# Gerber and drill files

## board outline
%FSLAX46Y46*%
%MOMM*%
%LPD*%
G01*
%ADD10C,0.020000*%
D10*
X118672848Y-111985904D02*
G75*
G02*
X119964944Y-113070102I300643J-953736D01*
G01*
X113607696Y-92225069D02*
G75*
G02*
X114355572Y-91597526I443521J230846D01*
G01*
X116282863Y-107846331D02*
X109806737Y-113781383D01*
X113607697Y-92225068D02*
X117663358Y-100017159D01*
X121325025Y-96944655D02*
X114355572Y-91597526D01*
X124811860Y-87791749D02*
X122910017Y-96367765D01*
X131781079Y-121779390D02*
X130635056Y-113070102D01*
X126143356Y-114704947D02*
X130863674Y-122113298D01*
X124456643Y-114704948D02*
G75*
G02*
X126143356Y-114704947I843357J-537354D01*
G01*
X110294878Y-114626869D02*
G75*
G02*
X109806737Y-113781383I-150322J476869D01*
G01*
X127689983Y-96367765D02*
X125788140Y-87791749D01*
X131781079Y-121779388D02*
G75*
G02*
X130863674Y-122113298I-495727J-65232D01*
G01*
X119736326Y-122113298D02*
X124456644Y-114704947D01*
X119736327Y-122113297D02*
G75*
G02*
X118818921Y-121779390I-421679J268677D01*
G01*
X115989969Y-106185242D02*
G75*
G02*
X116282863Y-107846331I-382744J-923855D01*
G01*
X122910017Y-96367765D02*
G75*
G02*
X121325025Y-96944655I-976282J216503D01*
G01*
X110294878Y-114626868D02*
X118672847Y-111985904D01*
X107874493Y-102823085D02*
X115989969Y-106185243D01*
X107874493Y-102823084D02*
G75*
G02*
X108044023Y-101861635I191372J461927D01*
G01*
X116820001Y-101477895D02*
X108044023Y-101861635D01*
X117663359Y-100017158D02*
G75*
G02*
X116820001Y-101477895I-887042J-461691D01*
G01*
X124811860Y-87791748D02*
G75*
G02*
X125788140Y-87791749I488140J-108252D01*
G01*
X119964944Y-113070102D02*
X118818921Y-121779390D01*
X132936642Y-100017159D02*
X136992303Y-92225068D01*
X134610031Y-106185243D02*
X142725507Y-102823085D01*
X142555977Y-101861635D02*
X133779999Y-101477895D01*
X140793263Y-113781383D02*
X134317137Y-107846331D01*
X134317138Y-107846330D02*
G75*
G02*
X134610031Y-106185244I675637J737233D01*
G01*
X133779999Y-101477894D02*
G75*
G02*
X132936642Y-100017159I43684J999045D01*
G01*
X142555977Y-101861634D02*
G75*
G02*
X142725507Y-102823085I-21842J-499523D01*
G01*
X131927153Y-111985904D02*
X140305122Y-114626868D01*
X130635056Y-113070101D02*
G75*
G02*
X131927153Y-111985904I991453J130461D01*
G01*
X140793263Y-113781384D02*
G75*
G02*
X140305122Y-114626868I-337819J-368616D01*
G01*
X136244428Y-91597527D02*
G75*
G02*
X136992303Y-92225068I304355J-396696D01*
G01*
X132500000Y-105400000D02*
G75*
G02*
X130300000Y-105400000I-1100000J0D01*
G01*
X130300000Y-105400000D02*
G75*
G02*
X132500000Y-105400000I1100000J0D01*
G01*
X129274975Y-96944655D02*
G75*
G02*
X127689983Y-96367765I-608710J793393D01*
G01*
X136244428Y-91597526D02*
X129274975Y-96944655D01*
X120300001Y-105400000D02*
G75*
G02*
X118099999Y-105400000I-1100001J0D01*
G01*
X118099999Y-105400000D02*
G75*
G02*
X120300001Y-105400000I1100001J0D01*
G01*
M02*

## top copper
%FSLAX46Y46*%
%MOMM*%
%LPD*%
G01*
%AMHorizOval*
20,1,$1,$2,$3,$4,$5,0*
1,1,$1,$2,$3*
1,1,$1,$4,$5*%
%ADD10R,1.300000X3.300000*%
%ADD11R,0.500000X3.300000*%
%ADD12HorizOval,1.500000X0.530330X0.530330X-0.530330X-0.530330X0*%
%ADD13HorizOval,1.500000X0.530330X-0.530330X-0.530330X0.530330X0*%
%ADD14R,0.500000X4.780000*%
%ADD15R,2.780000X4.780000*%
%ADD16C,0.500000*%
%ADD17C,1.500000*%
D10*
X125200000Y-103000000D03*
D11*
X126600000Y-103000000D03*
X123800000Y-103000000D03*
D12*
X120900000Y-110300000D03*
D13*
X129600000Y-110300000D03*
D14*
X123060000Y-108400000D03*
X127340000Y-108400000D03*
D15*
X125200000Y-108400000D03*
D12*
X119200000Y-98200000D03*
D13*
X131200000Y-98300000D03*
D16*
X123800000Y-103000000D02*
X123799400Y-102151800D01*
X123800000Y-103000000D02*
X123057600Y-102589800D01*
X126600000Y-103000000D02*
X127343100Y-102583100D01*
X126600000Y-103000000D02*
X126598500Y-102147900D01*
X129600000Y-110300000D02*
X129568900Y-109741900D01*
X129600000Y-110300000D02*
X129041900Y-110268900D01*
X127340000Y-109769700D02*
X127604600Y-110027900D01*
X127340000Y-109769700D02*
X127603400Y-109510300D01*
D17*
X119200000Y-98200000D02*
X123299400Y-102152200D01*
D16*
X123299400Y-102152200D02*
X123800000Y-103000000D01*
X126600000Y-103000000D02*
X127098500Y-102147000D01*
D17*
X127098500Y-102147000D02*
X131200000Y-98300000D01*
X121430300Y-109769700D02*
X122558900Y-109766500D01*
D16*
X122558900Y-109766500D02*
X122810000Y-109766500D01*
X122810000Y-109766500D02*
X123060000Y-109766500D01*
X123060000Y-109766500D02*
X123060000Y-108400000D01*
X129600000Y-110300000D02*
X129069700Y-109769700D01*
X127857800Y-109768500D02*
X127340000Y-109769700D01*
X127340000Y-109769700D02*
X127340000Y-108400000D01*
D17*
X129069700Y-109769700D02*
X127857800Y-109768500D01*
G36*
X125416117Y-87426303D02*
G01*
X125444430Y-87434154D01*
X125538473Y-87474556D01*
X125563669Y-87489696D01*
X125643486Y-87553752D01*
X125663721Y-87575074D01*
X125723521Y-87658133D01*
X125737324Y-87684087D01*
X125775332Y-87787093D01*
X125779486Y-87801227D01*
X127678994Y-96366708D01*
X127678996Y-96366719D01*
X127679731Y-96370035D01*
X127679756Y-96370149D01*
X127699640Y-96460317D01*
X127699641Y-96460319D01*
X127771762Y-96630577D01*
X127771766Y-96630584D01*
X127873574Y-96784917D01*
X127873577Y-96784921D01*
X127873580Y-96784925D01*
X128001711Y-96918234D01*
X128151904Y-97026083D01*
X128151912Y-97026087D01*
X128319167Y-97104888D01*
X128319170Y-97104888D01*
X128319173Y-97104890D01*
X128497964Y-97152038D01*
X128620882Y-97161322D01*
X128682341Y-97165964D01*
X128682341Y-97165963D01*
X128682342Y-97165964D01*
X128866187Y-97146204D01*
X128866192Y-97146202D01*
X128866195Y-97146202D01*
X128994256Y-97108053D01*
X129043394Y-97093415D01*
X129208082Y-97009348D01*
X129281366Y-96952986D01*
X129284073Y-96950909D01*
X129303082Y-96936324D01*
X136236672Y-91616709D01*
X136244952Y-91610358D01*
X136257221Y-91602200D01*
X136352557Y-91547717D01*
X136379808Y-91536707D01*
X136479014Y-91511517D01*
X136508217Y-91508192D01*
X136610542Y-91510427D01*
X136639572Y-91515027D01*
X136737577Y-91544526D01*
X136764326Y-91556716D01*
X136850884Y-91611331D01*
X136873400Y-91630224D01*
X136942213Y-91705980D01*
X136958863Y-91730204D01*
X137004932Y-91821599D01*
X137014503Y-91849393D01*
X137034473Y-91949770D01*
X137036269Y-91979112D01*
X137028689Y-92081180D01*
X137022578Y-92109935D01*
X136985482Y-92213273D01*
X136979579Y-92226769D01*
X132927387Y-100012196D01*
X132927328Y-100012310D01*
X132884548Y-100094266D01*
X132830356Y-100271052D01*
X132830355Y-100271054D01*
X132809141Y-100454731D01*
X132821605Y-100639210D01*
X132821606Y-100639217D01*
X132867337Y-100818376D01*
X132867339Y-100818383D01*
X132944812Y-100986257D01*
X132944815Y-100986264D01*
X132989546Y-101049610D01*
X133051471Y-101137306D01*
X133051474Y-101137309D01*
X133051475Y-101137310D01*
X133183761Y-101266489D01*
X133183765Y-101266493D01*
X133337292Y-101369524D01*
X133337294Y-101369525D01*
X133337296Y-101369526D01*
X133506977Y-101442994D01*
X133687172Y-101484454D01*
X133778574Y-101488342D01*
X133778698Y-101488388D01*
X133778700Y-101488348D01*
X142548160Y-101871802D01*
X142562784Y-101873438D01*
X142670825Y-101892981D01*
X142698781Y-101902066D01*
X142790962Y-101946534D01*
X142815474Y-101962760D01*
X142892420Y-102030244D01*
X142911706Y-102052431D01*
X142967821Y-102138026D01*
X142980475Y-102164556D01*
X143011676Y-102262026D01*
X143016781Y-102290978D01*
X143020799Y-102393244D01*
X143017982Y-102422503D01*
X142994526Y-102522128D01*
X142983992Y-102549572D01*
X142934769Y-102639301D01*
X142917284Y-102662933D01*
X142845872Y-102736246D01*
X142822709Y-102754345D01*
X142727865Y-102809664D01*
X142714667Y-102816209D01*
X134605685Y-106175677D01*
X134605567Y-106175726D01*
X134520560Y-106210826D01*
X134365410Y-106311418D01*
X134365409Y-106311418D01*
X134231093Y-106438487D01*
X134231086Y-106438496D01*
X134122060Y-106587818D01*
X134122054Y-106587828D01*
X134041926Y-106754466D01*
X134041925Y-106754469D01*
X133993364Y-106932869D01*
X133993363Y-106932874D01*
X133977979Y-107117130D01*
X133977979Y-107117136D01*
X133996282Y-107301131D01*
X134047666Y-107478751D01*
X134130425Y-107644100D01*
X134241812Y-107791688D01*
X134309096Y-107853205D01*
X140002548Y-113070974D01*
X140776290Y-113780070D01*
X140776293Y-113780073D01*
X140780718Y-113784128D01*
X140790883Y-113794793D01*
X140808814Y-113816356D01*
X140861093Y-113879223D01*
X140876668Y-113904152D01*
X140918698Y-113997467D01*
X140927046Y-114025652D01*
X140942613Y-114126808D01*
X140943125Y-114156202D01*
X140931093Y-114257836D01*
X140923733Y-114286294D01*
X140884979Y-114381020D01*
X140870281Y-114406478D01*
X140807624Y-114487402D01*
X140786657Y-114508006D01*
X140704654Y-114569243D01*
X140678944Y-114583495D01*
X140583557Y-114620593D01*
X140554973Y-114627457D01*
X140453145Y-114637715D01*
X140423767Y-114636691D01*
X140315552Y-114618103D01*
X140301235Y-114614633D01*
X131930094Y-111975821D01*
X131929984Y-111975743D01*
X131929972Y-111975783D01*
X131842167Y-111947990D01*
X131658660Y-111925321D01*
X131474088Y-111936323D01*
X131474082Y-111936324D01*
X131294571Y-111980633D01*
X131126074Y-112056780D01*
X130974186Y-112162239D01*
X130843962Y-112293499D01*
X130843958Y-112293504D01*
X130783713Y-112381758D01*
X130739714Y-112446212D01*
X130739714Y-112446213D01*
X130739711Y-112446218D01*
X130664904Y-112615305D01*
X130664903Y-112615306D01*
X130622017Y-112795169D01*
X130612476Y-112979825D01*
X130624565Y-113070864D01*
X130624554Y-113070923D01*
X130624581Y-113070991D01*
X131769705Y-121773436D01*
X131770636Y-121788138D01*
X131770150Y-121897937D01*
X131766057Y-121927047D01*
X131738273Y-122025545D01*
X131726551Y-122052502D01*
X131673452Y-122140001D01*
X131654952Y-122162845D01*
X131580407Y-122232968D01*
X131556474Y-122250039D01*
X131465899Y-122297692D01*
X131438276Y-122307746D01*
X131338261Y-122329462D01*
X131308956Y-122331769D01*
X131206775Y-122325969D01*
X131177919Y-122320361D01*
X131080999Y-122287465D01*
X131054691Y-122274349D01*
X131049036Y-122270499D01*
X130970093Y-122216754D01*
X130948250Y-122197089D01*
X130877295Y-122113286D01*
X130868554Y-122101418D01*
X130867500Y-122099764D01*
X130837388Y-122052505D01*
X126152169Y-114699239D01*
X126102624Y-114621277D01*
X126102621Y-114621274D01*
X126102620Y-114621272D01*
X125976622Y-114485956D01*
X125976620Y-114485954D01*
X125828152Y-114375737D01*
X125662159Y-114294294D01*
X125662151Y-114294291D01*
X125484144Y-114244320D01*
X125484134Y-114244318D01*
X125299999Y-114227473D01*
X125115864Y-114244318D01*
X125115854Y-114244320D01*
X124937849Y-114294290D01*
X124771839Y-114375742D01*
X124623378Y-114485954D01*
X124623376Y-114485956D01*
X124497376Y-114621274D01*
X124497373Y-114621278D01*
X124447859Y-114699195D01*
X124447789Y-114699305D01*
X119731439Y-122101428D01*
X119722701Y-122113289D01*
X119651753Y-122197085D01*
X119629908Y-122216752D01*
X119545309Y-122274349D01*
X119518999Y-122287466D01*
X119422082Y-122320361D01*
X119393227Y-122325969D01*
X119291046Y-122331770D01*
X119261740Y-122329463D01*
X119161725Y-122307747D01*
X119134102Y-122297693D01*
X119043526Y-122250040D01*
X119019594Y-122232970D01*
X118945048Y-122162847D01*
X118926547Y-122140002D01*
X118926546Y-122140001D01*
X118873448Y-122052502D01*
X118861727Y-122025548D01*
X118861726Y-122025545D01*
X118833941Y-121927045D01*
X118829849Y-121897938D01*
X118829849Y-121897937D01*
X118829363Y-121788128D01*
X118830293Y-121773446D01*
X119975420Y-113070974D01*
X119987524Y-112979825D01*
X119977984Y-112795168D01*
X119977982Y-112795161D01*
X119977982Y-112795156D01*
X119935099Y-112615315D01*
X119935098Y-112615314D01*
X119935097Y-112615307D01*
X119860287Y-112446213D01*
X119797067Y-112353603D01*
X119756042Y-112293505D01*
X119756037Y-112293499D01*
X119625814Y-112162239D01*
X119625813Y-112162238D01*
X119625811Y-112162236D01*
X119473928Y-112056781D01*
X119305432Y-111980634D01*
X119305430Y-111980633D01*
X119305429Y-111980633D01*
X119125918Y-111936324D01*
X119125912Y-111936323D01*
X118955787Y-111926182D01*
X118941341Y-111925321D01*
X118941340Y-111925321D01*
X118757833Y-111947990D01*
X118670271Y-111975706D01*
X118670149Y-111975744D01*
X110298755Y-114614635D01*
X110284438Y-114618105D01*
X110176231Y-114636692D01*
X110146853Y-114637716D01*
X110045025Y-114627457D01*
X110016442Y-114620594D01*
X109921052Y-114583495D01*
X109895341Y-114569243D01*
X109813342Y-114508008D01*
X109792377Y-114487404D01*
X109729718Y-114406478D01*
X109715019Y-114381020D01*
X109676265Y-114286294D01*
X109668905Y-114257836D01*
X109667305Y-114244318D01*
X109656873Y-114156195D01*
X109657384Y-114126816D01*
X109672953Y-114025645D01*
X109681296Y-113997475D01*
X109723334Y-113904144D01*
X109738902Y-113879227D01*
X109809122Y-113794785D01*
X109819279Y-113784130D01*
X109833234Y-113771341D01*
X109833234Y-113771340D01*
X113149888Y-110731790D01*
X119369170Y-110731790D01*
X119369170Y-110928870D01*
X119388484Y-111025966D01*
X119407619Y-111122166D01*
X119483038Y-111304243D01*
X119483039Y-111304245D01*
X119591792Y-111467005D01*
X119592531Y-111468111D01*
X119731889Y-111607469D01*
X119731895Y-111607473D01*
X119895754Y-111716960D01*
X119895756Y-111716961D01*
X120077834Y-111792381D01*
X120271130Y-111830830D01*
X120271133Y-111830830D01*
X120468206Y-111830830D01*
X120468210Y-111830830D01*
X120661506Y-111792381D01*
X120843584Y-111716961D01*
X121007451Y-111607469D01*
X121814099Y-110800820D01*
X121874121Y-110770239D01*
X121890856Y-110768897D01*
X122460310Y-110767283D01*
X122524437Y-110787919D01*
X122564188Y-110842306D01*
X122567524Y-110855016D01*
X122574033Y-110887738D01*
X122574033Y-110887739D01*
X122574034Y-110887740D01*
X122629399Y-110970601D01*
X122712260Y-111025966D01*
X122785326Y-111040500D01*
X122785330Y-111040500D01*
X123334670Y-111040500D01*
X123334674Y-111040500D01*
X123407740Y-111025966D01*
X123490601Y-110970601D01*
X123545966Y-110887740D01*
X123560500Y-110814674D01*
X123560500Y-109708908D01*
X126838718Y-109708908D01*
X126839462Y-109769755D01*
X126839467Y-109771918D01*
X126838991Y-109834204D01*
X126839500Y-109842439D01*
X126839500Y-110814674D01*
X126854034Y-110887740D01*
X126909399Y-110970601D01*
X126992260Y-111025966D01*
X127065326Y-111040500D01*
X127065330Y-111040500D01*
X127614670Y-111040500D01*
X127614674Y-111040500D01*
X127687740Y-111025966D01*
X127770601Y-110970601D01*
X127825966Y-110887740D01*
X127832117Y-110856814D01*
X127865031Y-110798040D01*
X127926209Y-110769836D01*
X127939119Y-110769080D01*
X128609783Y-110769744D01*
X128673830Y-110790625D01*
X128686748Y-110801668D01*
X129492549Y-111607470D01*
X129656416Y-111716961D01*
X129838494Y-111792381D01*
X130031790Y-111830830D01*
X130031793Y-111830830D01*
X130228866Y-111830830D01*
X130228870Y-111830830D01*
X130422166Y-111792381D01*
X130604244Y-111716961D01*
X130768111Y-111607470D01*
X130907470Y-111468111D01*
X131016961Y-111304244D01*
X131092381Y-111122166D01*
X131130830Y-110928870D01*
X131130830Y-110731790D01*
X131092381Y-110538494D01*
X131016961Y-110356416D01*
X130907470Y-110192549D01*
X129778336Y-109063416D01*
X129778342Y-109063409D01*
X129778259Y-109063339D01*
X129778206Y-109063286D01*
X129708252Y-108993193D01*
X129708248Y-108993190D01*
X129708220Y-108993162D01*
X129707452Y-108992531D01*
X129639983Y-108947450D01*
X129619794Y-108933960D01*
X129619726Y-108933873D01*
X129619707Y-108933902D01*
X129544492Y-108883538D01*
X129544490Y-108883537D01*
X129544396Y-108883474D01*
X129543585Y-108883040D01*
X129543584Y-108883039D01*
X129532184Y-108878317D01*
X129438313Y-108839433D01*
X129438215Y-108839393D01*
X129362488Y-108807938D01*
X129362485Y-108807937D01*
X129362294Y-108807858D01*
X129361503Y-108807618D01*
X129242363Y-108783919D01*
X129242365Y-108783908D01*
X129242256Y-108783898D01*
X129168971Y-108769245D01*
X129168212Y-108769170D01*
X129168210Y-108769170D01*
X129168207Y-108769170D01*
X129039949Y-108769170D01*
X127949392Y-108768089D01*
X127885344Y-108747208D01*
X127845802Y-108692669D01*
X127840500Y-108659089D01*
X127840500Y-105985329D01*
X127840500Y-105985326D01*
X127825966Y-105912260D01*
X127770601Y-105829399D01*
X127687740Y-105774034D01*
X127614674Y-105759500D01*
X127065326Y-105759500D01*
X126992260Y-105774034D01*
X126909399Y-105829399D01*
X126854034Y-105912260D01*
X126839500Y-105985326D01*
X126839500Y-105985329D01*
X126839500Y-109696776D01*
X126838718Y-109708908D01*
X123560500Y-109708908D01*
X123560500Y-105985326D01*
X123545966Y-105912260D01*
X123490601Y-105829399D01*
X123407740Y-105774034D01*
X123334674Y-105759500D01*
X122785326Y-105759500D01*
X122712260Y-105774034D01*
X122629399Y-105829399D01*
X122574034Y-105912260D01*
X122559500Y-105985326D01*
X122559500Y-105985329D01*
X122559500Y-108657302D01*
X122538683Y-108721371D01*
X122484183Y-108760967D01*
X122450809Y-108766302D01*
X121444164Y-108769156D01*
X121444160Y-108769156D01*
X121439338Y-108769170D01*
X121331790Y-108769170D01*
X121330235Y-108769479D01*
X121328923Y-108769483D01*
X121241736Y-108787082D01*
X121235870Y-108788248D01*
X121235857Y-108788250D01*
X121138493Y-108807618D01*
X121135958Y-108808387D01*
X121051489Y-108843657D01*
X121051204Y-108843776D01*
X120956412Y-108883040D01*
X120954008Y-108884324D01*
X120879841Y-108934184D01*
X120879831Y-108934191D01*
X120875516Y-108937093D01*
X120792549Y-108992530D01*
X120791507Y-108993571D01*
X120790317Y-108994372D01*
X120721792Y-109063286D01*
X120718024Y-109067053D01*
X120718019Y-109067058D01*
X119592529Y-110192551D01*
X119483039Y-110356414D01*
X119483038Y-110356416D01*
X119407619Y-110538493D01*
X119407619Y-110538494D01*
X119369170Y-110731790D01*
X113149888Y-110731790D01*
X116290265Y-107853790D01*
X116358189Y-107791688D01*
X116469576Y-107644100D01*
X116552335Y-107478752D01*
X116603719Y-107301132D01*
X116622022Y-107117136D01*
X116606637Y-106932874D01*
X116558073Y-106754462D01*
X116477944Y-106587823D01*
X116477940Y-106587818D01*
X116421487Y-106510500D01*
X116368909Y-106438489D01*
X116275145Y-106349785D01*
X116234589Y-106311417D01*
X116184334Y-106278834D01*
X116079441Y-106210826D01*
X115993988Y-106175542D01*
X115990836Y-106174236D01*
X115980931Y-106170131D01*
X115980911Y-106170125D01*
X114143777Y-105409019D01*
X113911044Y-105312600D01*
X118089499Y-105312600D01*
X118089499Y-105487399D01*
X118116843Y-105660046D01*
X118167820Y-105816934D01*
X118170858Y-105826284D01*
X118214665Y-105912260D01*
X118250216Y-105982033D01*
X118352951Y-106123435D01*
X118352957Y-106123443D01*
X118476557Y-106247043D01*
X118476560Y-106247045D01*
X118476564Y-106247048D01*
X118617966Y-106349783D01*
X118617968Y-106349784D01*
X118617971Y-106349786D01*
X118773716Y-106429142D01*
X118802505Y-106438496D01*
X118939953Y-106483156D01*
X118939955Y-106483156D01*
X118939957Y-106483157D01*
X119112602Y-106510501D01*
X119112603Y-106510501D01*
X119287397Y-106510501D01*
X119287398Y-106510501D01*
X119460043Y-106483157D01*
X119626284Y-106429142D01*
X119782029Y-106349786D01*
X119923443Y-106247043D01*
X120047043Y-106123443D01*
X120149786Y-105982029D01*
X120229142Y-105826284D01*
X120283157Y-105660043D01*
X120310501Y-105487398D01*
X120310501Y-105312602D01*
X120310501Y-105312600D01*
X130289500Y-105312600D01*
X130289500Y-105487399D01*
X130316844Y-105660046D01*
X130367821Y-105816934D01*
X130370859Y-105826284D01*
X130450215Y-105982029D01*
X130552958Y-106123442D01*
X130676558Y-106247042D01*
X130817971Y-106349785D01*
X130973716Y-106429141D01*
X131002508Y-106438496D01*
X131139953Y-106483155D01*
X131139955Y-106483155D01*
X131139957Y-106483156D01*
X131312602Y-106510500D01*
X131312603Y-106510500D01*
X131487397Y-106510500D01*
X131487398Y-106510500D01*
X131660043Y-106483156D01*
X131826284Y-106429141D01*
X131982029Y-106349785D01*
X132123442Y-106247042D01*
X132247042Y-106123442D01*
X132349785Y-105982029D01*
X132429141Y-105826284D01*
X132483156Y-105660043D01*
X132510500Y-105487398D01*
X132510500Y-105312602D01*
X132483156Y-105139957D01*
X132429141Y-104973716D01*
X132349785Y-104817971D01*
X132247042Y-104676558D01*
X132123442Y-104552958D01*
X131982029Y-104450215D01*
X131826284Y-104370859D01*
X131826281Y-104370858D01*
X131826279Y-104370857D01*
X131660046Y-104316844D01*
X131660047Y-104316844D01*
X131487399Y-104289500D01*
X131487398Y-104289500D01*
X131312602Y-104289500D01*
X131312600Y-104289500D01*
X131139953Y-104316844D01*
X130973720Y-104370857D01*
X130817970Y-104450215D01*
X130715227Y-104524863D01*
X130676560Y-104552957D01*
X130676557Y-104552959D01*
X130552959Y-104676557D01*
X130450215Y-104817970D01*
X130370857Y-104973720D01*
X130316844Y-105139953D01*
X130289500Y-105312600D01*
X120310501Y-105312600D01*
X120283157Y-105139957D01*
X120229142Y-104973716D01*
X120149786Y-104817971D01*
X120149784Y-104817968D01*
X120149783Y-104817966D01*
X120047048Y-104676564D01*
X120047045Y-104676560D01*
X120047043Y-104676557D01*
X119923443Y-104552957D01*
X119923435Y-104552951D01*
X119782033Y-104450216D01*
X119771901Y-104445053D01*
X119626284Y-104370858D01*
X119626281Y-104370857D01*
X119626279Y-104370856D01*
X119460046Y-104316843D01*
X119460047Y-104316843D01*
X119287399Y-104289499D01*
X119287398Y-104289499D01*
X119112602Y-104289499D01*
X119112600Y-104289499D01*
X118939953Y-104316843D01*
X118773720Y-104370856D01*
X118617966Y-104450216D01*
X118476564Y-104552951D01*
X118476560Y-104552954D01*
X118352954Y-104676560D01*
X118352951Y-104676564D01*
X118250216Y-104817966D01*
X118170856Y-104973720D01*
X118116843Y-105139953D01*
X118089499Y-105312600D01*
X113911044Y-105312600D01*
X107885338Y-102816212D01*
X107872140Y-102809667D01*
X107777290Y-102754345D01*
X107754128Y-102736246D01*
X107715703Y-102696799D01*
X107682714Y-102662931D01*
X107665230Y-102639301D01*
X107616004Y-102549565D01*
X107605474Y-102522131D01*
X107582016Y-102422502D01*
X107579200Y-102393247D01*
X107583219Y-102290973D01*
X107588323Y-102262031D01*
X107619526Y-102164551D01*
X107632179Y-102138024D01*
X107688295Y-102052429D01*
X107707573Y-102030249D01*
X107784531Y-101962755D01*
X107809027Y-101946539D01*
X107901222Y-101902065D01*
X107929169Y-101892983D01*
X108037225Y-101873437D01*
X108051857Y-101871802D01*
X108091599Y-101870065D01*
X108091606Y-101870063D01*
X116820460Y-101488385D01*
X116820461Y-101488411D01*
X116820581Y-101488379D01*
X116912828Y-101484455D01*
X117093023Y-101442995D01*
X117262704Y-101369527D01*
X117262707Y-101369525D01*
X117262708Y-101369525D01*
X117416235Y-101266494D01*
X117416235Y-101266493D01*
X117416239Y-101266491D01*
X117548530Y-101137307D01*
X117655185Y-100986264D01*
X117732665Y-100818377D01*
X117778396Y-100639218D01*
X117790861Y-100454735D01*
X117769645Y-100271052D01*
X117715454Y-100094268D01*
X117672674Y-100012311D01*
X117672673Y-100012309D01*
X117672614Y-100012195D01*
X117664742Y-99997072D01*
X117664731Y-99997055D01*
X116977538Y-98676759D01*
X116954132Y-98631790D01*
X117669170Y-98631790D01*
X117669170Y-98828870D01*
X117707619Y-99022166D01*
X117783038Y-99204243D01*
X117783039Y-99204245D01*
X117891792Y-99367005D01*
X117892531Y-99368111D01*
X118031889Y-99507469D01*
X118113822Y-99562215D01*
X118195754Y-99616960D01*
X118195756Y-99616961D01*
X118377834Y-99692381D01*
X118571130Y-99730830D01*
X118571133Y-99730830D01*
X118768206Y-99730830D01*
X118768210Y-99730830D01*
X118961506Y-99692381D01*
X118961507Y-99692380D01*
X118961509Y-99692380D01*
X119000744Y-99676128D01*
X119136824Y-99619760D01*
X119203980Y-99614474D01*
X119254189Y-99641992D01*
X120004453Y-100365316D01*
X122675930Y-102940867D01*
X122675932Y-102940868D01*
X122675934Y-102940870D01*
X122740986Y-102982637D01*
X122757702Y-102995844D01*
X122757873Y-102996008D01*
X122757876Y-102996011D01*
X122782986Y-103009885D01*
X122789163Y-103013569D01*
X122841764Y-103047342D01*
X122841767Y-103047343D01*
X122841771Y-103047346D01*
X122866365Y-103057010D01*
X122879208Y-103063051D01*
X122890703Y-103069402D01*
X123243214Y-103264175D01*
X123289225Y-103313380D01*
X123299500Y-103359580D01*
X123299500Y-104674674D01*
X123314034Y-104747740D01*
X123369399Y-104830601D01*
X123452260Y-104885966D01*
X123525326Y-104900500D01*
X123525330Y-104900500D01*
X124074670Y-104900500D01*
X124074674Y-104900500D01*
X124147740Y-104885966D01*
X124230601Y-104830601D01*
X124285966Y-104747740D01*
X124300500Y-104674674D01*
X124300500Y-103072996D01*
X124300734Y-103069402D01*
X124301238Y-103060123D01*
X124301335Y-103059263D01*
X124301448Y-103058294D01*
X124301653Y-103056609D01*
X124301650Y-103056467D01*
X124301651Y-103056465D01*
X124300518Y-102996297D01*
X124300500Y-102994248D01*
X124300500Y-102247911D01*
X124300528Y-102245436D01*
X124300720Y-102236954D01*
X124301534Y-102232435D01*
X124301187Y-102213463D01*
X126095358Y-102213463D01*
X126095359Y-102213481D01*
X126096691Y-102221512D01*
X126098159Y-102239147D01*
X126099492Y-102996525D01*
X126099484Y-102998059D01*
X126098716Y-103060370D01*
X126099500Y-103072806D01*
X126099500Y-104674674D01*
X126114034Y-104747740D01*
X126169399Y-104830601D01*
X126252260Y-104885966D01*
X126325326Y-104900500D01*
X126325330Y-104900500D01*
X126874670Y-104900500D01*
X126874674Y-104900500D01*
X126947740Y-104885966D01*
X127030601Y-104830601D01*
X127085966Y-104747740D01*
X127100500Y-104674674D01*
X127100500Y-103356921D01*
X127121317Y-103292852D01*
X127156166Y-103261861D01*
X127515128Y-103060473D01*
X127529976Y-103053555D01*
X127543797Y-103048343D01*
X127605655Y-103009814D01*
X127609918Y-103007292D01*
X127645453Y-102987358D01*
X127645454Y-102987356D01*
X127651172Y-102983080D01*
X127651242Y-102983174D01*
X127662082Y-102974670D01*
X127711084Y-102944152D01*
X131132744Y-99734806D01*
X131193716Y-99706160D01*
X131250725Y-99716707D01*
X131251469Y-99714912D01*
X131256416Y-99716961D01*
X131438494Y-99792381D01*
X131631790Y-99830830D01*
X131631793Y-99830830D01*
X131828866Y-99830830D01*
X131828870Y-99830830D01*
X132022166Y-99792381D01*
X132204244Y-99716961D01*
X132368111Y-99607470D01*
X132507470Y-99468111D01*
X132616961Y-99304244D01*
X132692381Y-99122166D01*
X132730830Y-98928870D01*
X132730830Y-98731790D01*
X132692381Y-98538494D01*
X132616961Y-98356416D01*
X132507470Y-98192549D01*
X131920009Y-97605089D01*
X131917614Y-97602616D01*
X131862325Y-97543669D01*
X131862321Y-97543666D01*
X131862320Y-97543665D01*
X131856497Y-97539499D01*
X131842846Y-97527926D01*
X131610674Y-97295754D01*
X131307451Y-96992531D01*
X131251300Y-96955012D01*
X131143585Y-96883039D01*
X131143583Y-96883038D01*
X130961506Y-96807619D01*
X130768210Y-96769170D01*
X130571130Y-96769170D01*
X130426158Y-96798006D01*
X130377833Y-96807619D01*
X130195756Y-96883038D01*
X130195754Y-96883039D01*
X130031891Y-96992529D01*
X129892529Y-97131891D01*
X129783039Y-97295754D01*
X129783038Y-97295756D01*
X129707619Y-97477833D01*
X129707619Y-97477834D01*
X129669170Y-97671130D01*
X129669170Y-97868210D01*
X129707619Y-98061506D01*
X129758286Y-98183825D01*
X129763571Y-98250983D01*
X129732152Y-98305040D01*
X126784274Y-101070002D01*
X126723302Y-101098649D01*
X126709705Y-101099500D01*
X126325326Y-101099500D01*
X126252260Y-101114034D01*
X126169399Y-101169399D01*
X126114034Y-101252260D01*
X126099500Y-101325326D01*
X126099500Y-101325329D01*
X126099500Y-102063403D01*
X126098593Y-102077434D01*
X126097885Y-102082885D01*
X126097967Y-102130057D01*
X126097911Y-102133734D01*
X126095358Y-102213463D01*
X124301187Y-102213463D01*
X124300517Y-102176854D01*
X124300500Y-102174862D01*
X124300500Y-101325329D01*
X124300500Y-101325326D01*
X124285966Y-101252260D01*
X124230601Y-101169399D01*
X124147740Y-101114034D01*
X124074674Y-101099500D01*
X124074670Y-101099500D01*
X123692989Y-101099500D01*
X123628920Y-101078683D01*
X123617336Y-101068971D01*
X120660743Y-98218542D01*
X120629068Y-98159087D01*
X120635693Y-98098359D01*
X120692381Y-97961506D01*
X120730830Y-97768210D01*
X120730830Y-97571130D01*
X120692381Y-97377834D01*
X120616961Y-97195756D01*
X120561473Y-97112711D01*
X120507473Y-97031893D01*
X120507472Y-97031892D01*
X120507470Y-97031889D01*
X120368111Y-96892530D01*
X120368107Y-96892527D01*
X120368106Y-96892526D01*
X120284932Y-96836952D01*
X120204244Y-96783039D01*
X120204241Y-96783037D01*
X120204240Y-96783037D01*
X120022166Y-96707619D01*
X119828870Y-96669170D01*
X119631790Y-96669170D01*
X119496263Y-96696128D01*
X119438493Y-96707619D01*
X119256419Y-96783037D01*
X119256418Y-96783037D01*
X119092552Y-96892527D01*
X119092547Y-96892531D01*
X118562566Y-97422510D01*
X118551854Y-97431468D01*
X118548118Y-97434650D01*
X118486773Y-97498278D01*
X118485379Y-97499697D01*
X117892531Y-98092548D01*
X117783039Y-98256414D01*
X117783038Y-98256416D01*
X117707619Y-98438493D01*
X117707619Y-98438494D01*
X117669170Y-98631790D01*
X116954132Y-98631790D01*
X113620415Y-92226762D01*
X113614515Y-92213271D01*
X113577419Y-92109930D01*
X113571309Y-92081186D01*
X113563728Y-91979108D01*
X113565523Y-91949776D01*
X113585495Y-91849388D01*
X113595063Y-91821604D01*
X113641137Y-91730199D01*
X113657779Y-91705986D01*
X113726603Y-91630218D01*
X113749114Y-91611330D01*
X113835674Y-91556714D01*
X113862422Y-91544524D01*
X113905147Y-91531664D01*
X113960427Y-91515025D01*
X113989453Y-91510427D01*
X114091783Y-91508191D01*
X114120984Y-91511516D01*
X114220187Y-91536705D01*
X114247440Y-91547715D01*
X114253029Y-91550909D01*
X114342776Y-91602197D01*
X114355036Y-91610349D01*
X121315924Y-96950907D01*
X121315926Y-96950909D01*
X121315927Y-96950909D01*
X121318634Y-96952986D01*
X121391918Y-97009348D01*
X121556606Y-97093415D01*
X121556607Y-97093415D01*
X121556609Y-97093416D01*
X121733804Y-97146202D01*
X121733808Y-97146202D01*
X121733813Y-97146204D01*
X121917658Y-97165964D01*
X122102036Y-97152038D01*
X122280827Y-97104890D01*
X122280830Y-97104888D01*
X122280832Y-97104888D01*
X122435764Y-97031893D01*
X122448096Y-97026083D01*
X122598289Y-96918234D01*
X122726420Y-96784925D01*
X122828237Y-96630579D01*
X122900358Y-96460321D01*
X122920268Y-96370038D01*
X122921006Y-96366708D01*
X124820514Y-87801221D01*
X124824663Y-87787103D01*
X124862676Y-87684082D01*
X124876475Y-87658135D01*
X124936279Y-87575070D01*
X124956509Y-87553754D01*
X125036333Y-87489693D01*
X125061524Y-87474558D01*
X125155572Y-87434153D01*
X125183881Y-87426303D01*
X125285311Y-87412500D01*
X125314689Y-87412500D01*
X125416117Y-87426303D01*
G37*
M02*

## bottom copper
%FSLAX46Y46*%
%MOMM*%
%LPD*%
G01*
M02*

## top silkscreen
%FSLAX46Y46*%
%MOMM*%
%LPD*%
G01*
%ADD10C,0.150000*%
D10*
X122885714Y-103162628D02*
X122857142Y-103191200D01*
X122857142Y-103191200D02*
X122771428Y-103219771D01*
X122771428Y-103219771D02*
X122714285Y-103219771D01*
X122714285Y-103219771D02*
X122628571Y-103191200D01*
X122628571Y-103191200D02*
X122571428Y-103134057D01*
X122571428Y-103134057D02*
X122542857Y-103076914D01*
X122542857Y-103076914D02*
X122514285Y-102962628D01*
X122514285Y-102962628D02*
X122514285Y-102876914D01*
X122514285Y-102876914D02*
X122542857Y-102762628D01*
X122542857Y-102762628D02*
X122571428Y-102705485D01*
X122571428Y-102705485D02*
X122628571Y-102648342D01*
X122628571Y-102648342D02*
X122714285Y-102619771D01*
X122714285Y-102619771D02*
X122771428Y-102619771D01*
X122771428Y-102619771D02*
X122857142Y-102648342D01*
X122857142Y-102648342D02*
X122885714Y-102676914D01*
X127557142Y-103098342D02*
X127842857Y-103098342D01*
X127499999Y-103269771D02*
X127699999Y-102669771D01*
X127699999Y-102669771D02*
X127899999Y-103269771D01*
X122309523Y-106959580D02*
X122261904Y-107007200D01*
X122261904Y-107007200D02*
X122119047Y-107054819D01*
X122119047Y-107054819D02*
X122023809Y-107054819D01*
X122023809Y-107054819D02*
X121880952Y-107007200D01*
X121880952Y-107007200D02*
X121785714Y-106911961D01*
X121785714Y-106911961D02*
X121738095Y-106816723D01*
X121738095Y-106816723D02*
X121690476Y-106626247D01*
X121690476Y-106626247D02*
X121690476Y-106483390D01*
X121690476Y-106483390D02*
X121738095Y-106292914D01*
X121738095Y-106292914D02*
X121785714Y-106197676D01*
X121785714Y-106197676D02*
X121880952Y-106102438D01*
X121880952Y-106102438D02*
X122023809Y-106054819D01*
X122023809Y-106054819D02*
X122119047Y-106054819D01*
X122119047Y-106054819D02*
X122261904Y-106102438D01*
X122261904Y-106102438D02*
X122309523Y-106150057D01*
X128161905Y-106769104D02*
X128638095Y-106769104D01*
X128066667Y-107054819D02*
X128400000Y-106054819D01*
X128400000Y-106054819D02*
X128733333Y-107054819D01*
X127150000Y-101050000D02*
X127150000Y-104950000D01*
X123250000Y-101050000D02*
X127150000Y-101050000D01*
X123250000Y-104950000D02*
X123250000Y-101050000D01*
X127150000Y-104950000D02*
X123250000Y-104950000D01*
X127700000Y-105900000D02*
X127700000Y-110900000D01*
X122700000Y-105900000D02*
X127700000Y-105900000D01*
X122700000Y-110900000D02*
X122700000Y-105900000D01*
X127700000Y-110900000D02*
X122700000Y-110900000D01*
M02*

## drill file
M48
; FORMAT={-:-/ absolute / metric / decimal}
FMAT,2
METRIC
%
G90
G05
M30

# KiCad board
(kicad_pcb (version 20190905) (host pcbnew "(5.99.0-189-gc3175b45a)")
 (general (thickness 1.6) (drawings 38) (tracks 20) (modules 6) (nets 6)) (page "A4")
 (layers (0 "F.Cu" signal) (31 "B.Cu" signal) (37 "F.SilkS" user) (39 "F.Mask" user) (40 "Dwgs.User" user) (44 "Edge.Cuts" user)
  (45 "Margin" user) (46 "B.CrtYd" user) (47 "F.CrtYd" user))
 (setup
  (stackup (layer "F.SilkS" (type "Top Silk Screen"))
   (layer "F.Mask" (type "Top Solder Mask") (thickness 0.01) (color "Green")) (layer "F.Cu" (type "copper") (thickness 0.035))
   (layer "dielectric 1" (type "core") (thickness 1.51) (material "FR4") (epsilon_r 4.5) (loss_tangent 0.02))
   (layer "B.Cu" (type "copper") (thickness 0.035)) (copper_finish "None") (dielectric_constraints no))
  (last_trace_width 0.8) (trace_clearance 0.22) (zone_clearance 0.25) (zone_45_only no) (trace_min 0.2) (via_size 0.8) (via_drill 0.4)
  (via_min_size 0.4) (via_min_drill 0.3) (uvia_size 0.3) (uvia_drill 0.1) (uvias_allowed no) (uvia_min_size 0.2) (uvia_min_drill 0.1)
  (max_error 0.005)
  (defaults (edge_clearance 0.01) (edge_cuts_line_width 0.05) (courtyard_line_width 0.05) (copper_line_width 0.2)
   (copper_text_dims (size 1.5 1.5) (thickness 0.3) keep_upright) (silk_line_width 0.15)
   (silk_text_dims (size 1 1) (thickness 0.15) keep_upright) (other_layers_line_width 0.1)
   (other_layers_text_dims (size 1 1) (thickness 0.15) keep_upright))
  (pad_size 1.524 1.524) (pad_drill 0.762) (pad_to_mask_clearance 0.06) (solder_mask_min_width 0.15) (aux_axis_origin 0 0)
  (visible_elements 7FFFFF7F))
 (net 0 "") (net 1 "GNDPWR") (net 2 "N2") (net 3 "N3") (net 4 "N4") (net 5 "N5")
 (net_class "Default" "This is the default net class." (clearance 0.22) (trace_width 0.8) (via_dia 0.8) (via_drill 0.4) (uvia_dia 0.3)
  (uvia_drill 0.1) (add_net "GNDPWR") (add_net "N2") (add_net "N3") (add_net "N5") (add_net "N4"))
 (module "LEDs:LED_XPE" (layer "F.Cu") (at 125.2 103 180)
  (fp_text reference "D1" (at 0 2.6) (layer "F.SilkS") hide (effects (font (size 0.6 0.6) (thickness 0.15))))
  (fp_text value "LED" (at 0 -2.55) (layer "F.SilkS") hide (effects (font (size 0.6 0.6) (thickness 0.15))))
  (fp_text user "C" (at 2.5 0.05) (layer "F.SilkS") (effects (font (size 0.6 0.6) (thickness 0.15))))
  (fp_line (start -1.95 1.95) (end -1.95 -1.95) (layer "F.SilkS") (width 0.15))
  (fp_line (start 1.95 1.95) (end -1.95 1.95) (layer "F.SilkS") (width 0.15))
  (fp_line (start 1.95 -1.95) (end 1.95 1.95) (layer "F.SilkS") (width 0.15))
  (fp_line (start -1.95 -1.95) (end 1.95 -1.95) (layer "F.SilkS") (width 0.15))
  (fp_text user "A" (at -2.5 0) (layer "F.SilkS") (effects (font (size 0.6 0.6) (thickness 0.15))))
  (pad "PAD" smd rect (at 0 0 180) (size 1.3 3.3) (layers "F.Cu" "F.Paste" "F.Mask") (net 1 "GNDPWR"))
  (pad "A" smd rect (at -1.4 0 180) (size 0.5 3.3) (layers "F.Cu" "F.Paste" "F.Mask") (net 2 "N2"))
  (pad "C" smd rect (at 1.4 0 180) (size 0.5 3.3) (layers "F.Cu" "F.Paste" "F.Mask") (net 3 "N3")))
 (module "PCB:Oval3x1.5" (layer "F.Cu") (at 120.9 110.3 45)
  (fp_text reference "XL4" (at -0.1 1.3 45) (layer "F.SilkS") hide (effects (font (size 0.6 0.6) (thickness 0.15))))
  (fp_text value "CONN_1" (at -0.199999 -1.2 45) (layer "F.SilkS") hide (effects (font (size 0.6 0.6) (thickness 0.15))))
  (pad "1" smd oval (at 0 0 45) (size 3 1.5) (layers "F.Cu" "F.Paste" "F.Mask") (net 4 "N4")))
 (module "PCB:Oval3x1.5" (layer "F.Cu") (at 129.6 110.3 -45)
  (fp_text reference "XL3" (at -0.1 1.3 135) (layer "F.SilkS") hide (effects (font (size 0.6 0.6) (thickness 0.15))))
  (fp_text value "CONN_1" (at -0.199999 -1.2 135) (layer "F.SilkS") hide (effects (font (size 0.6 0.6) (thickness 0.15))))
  (pad "1" smd oval (at 0 0 315) (size 3 1.5) (layers "F.Cu" "F.Paste" "F.Mask") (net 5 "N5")))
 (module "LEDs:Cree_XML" (layer "F.Cu") (at 125.2 108.4 180)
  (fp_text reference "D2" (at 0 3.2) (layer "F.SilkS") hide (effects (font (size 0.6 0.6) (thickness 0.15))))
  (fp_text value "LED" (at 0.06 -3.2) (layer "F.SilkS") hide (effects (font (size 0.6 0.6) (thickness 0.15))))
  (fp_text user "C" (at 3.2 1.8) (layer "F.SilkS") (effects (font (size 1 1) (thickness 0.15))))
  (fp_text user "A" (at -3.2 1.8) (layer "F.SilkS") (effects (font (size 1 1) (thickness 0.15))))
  (fp_line (start -2.5 2.5) (end -2.5 -2.5) (layer "F.SilkS") (width 0.15))
  (fp_line (start 2.5 2.5) (end -2.5 2.5) (layer "F.SilkS") (width 0.15))
  (fp_line (start 2.5 -2.5) (end 2.5 2.5) (layer "F.SilkS") (width 0.15))
  (fp_line (start -2.5 -2.5) (end 2.5 -2.5) (layer "F.SilkS") (width 0.15))
  (pad "C" smd rect (at 2.14 0 180) (size 0.5 4.78) (layers "F.Cu" "F.Paste" "F.Mask") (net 4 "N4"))
  (pad "A" smd rect (at -2.14 0 180) (size 0.5 4.78) (layers "F.Cu" "F.Paste" "F.Mask") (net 5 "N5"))
  (pad "PAD" smd rect (at 0 0 180) (size 2.78 4.78) (layers "F.Cu" "F.Paste" "F.Mask") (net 1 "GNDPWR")))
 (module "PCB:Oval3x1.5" (layer "F.Cu") (at 119.2 98.2 45)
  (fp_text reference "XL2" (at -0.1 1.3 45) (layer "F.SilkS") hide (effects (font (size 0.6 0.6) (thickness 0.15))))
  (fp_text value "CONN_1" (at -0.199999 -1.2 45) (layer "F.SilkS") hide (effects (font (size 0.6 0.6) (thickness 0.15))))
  (pad "1" smd oval (at 0 0 45) (size 3 1.5) (layers "F.Cu" "F.Paste" "F.Mask") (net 3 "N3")))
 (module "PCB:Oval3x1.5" (layer "F.Cu") (at 131.2 98.3 -45)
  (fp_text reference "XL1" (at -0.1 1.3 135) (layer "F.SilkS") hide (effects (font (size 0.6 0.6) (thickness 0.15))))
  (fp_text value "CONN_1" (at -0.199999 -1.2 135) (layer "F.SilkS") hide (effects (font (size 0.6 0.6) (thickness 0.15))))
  (pad "1" smd oval (at 0 0 315) (size 3 1.5) (layers "F.Cu" "F.Paste" "F.Mask") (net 2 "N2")))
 (gr_arc (start 118.973491 112.93964) (end 119.964944 113.070102) (angle -114.9925404) (layer "Edge.Cuts") (width 0.02))
 (gr_arc (start 114.051217 91.994223) (end 114.355572 91.597526) (angle -154.9925404) (layer "Edge.Cuts") (width 0.02))
 (gr_line (start 116.282863 107.846331) (end 109.806737 113.781383) (layer "Edge.Cuts") (width 0.02))
 (gr_line (start 113.607697 92.225068) (end 117.663358 100.017159) (layer "Edge.Cuts") (width 0.02))
 (gr_line (start 121.325025 96.944655) (end 114.355572 91.597526) (layer "Edge.Cuts") (width 0.02))
 (gr_line (start 124.81186 87.791749) (end 122.910017 96.367765) (layer "Edge.Cuts") (width 0.02))
 (gr_line (start 131.781079 121.77939) (end 130.635056 113.070102) (layer "Edge.Cuts") (width 0.02))
 (gr_line (start 126.143356 114.704947) (end 130.863674 122.113298) (layer "Edge.Cuts") (width 0.02))
 (gr_arc (start 125.3 115.242302) (end 126.143356 114.704947) (angle -114.9925404) (layer "Edge.Cuts") (width 0.02))
 (gr_arc (start 110.144556 114.15) (end 109.806737 113.781383) (angle -154.9925404) (layer "Edge.Cuts") (width 0.02))
 (gr_line (start 127.689983 96.367765) (end 125.78814 87.791749) (layer "Edge.Cuts") (width 0.02))
 (gr_arc (start 131.285352 121.84462) (end 130.863674 122.113298) (angle -154.9925404) (layer "Edge.Cuts") (width 0.02))
 (gr_line (start 119.736326 122.113298) (end 124.456644 114.704947) (layer "Edge.Cuts") (width 0.02))
 (gr_arc (start 119.314648 121.84462) (end 118.818921 121.77939) (angle -154.9925404) (layer "Edge.Cuts") (width 0.02))
 (gr_arc (start 115.607225 107.109097) (end 116.282863 107.846331) (angle -114.9925404) (layer "Edge.Cuts") (width 0.02))
 (gr_arc (start 121.933735 96.151262) (end 121.325025 96.944655) (angle -114.9925404) (layer "Edge.Cuts") (width 0.02))
 (gr_line (start 110.294878 114.626868) (end 118.672847 111.985904) (layer "Edge.Cuts") (width 0.02))
 (gr_line (start 107.874493 102.823085) (end 115.989969 106.185243) (layer "Edge.Cuts") (width 0.02))
 (gr_arc (start 108.065865 102.361157) (end 108.044023 101.861635) (angle -154.9925404) (layer "Edge.Cuts") (width 0.02))
 (gr_line (start 116.820001 101.477895) (end 108.044023 101.861635) (layer "Edge.Cuts") (width 0.02))
 (gr_arc (start 116.776317 100.478849) (end 116.820001 101.477895) (angle -114.9925404) (layer "Edge.Cuts") (width 0.02))
 (gr_arc (start 125.3 87.9) (end 125.78814 87.791749) (angle -154.9925404) (layer "Edge.Cuts") (width 0.02))
 (gr_line (start 119.964944 113.070102) (end 118.818921 121.77939) (layer "Edge.Cuts") (width 0.02))
 (gr_line (start 132.936642 100.017159) (end 136.992303 92.225068) (layer "Edge.Cuts") (width 0.02))
 (gr_line (start 134.610031 106.185243) (end 142.725507 102.823085) (layer "Edge.Cuts") (width 0.02))
 (gr_line (start 142.555977 101.861635) (end 133.779999 101.477895) (layer "Edge.Cuts") (width 0.02))
 (gr_line (start 140.793263 113.781383) (end 134.317137 107.846331) (layer "Edge.Cuts") (width 0.02))
 (gr_arc (start 134.992775 107.109097) (end 134.610031 106.185243) (angle -114.9925404) (layer "Edge.Cuts") (width 0.02))
 (gr_arc (start 133.823683 100.478849) (end 132.936642 100.017159) (angle -114.9925404) (layer "Edge.Cuts") (width 0.02))
 (gr_arc (start 142.534135 102.361157) (end 142.725507 102.823085) (angle -154.9925404) (layer "Edge.Cuts") (width 0.02))
 (gr_line (start 131.927153 111.985904) (end 140.305122 114.626868) (layer "Edge.Cuts") (width 0.02))
 (gr_arc (start 131.626509 112.93964) (end 131.927153 111.985904) (angle -114.9925404) (layer "Edge.Cuts") (width 0.02))
 (gr_arc (start 140.455444 114.15) (end 140.305122 114.626868) (angle -154.9925404) (layer "Edge.Cuts") (width 0.02))
 (gr_arc (start 136.548783 91.994223) (end 136.992303 92.225068) (angle -154.9925404) (layer "Edge.Cuts") (width 0.02))
 (gr_circle (center 131.4 105.4) (end 132.5 105.4) (layer "Edge.Cuts") (width 0.02))
 (gr_arc (start 128.666265 96.151262) (end 127.689983 96.367765) (angle -114.9925404) (layer "Edge.Cuts") (width 0.02))
 (gr_line (start 136.244428 91.597526) (end 129.274975 96.944655) (layer "Edge.Cuts") (width 0.02))
 (gr_circle (center 119.2 105.4) (end 120.300001 105.4) (layer "Edge.Cuts") (width 0.02))
 (segment (start 123.8 103) (end 123.7994 102.1518) (width 0.5) (layer "F.Cu") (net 3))
 (segment (start 123.8 103) (end 123.0576 102.5898) (width 0.5) (layer "F.Cu") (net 3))
 (segment (start 126.6 103) (end 127.3431 102.5831) (width 0.5) (layer "F.Cu") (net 2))
 (segment (start 126.6 103) (end 126.5985 102.1479) (width 0.5) (layer "F.Cu") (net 2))
 (segment (start 129.6 110.3) (end 129.5689 109.7419) (width 0.5) (layer "F.Cu") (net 5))
 (segment (start 129.6 110.3) (end 129.0419 110.2689) (width 0.5) (layer "F.Cu") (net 5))
 (segment (start 127.34 109.7697) (end 127.6046 110.0279) (width 0.5) (layer "F.Cu") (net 5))
 (segment (start 127.34 109.7697) (end 127.6034 109.5103) (width 0.5) (layer "F.Cu") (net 5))
 (segment (start 119.2 98.2) (end 123.2994 102.1522) (width 1.5) (layer "F.Cu") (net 3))
 (segment (start 123.2994 102.1522) (end 123.8 103) (width 0.5) (layer "F.Cu") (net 3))
 (segment (start 126.6 103) (end 127.0985 102.147) (width 0.5) (layer "F.Cu") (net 2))
 (segment (start 127.0985 102.147) (end 131.2 98.3) (width 1.5) (layer "F.Cu") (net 2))
 (segment (start 121.4303 109.7697) (end 122.5589 109.7665) (width 1.5) (layer "F.Cu") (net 4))
 (segment (start 122.5589 109.7665) (end 122.81 109.7665) (width 0.5) (layer "F.Cu") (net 4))
 (segment (start 122.81 109.7665) (end 123.06 109.7665) (width 0.5) (layer "F.Cu") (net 4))
 (segment (start 123.06 109.7665) (end 123.06 108.4) (width 0.5) (layer "F.Cu") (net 4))
 (segment (start 129.6 110.3) (end 129.0697 109.7697) (width 0.5) (layer "F.Cu") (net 5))
 (segment (start 127.8578 109.7685) (end 127.34 109.7697) (width 0.5) (layer "F.Cu") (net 5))
 (segment (start 127.34 109.7697) (end 127.34 108.4) (width 0.5) (layer "F.Cu") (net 5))
 (segment (start 129.0697 109.7697) (end 127.8578 109.7685) (width 1.5) (layer "F.Cu") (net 5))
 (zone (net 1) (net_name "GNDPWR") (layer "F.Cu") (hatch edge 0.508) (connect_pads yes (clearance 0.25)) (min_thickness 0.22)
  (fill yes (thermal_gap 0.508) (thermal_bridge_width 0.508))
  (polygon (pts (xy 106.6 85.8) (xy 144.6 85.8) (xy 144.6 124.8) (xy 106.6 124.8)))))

